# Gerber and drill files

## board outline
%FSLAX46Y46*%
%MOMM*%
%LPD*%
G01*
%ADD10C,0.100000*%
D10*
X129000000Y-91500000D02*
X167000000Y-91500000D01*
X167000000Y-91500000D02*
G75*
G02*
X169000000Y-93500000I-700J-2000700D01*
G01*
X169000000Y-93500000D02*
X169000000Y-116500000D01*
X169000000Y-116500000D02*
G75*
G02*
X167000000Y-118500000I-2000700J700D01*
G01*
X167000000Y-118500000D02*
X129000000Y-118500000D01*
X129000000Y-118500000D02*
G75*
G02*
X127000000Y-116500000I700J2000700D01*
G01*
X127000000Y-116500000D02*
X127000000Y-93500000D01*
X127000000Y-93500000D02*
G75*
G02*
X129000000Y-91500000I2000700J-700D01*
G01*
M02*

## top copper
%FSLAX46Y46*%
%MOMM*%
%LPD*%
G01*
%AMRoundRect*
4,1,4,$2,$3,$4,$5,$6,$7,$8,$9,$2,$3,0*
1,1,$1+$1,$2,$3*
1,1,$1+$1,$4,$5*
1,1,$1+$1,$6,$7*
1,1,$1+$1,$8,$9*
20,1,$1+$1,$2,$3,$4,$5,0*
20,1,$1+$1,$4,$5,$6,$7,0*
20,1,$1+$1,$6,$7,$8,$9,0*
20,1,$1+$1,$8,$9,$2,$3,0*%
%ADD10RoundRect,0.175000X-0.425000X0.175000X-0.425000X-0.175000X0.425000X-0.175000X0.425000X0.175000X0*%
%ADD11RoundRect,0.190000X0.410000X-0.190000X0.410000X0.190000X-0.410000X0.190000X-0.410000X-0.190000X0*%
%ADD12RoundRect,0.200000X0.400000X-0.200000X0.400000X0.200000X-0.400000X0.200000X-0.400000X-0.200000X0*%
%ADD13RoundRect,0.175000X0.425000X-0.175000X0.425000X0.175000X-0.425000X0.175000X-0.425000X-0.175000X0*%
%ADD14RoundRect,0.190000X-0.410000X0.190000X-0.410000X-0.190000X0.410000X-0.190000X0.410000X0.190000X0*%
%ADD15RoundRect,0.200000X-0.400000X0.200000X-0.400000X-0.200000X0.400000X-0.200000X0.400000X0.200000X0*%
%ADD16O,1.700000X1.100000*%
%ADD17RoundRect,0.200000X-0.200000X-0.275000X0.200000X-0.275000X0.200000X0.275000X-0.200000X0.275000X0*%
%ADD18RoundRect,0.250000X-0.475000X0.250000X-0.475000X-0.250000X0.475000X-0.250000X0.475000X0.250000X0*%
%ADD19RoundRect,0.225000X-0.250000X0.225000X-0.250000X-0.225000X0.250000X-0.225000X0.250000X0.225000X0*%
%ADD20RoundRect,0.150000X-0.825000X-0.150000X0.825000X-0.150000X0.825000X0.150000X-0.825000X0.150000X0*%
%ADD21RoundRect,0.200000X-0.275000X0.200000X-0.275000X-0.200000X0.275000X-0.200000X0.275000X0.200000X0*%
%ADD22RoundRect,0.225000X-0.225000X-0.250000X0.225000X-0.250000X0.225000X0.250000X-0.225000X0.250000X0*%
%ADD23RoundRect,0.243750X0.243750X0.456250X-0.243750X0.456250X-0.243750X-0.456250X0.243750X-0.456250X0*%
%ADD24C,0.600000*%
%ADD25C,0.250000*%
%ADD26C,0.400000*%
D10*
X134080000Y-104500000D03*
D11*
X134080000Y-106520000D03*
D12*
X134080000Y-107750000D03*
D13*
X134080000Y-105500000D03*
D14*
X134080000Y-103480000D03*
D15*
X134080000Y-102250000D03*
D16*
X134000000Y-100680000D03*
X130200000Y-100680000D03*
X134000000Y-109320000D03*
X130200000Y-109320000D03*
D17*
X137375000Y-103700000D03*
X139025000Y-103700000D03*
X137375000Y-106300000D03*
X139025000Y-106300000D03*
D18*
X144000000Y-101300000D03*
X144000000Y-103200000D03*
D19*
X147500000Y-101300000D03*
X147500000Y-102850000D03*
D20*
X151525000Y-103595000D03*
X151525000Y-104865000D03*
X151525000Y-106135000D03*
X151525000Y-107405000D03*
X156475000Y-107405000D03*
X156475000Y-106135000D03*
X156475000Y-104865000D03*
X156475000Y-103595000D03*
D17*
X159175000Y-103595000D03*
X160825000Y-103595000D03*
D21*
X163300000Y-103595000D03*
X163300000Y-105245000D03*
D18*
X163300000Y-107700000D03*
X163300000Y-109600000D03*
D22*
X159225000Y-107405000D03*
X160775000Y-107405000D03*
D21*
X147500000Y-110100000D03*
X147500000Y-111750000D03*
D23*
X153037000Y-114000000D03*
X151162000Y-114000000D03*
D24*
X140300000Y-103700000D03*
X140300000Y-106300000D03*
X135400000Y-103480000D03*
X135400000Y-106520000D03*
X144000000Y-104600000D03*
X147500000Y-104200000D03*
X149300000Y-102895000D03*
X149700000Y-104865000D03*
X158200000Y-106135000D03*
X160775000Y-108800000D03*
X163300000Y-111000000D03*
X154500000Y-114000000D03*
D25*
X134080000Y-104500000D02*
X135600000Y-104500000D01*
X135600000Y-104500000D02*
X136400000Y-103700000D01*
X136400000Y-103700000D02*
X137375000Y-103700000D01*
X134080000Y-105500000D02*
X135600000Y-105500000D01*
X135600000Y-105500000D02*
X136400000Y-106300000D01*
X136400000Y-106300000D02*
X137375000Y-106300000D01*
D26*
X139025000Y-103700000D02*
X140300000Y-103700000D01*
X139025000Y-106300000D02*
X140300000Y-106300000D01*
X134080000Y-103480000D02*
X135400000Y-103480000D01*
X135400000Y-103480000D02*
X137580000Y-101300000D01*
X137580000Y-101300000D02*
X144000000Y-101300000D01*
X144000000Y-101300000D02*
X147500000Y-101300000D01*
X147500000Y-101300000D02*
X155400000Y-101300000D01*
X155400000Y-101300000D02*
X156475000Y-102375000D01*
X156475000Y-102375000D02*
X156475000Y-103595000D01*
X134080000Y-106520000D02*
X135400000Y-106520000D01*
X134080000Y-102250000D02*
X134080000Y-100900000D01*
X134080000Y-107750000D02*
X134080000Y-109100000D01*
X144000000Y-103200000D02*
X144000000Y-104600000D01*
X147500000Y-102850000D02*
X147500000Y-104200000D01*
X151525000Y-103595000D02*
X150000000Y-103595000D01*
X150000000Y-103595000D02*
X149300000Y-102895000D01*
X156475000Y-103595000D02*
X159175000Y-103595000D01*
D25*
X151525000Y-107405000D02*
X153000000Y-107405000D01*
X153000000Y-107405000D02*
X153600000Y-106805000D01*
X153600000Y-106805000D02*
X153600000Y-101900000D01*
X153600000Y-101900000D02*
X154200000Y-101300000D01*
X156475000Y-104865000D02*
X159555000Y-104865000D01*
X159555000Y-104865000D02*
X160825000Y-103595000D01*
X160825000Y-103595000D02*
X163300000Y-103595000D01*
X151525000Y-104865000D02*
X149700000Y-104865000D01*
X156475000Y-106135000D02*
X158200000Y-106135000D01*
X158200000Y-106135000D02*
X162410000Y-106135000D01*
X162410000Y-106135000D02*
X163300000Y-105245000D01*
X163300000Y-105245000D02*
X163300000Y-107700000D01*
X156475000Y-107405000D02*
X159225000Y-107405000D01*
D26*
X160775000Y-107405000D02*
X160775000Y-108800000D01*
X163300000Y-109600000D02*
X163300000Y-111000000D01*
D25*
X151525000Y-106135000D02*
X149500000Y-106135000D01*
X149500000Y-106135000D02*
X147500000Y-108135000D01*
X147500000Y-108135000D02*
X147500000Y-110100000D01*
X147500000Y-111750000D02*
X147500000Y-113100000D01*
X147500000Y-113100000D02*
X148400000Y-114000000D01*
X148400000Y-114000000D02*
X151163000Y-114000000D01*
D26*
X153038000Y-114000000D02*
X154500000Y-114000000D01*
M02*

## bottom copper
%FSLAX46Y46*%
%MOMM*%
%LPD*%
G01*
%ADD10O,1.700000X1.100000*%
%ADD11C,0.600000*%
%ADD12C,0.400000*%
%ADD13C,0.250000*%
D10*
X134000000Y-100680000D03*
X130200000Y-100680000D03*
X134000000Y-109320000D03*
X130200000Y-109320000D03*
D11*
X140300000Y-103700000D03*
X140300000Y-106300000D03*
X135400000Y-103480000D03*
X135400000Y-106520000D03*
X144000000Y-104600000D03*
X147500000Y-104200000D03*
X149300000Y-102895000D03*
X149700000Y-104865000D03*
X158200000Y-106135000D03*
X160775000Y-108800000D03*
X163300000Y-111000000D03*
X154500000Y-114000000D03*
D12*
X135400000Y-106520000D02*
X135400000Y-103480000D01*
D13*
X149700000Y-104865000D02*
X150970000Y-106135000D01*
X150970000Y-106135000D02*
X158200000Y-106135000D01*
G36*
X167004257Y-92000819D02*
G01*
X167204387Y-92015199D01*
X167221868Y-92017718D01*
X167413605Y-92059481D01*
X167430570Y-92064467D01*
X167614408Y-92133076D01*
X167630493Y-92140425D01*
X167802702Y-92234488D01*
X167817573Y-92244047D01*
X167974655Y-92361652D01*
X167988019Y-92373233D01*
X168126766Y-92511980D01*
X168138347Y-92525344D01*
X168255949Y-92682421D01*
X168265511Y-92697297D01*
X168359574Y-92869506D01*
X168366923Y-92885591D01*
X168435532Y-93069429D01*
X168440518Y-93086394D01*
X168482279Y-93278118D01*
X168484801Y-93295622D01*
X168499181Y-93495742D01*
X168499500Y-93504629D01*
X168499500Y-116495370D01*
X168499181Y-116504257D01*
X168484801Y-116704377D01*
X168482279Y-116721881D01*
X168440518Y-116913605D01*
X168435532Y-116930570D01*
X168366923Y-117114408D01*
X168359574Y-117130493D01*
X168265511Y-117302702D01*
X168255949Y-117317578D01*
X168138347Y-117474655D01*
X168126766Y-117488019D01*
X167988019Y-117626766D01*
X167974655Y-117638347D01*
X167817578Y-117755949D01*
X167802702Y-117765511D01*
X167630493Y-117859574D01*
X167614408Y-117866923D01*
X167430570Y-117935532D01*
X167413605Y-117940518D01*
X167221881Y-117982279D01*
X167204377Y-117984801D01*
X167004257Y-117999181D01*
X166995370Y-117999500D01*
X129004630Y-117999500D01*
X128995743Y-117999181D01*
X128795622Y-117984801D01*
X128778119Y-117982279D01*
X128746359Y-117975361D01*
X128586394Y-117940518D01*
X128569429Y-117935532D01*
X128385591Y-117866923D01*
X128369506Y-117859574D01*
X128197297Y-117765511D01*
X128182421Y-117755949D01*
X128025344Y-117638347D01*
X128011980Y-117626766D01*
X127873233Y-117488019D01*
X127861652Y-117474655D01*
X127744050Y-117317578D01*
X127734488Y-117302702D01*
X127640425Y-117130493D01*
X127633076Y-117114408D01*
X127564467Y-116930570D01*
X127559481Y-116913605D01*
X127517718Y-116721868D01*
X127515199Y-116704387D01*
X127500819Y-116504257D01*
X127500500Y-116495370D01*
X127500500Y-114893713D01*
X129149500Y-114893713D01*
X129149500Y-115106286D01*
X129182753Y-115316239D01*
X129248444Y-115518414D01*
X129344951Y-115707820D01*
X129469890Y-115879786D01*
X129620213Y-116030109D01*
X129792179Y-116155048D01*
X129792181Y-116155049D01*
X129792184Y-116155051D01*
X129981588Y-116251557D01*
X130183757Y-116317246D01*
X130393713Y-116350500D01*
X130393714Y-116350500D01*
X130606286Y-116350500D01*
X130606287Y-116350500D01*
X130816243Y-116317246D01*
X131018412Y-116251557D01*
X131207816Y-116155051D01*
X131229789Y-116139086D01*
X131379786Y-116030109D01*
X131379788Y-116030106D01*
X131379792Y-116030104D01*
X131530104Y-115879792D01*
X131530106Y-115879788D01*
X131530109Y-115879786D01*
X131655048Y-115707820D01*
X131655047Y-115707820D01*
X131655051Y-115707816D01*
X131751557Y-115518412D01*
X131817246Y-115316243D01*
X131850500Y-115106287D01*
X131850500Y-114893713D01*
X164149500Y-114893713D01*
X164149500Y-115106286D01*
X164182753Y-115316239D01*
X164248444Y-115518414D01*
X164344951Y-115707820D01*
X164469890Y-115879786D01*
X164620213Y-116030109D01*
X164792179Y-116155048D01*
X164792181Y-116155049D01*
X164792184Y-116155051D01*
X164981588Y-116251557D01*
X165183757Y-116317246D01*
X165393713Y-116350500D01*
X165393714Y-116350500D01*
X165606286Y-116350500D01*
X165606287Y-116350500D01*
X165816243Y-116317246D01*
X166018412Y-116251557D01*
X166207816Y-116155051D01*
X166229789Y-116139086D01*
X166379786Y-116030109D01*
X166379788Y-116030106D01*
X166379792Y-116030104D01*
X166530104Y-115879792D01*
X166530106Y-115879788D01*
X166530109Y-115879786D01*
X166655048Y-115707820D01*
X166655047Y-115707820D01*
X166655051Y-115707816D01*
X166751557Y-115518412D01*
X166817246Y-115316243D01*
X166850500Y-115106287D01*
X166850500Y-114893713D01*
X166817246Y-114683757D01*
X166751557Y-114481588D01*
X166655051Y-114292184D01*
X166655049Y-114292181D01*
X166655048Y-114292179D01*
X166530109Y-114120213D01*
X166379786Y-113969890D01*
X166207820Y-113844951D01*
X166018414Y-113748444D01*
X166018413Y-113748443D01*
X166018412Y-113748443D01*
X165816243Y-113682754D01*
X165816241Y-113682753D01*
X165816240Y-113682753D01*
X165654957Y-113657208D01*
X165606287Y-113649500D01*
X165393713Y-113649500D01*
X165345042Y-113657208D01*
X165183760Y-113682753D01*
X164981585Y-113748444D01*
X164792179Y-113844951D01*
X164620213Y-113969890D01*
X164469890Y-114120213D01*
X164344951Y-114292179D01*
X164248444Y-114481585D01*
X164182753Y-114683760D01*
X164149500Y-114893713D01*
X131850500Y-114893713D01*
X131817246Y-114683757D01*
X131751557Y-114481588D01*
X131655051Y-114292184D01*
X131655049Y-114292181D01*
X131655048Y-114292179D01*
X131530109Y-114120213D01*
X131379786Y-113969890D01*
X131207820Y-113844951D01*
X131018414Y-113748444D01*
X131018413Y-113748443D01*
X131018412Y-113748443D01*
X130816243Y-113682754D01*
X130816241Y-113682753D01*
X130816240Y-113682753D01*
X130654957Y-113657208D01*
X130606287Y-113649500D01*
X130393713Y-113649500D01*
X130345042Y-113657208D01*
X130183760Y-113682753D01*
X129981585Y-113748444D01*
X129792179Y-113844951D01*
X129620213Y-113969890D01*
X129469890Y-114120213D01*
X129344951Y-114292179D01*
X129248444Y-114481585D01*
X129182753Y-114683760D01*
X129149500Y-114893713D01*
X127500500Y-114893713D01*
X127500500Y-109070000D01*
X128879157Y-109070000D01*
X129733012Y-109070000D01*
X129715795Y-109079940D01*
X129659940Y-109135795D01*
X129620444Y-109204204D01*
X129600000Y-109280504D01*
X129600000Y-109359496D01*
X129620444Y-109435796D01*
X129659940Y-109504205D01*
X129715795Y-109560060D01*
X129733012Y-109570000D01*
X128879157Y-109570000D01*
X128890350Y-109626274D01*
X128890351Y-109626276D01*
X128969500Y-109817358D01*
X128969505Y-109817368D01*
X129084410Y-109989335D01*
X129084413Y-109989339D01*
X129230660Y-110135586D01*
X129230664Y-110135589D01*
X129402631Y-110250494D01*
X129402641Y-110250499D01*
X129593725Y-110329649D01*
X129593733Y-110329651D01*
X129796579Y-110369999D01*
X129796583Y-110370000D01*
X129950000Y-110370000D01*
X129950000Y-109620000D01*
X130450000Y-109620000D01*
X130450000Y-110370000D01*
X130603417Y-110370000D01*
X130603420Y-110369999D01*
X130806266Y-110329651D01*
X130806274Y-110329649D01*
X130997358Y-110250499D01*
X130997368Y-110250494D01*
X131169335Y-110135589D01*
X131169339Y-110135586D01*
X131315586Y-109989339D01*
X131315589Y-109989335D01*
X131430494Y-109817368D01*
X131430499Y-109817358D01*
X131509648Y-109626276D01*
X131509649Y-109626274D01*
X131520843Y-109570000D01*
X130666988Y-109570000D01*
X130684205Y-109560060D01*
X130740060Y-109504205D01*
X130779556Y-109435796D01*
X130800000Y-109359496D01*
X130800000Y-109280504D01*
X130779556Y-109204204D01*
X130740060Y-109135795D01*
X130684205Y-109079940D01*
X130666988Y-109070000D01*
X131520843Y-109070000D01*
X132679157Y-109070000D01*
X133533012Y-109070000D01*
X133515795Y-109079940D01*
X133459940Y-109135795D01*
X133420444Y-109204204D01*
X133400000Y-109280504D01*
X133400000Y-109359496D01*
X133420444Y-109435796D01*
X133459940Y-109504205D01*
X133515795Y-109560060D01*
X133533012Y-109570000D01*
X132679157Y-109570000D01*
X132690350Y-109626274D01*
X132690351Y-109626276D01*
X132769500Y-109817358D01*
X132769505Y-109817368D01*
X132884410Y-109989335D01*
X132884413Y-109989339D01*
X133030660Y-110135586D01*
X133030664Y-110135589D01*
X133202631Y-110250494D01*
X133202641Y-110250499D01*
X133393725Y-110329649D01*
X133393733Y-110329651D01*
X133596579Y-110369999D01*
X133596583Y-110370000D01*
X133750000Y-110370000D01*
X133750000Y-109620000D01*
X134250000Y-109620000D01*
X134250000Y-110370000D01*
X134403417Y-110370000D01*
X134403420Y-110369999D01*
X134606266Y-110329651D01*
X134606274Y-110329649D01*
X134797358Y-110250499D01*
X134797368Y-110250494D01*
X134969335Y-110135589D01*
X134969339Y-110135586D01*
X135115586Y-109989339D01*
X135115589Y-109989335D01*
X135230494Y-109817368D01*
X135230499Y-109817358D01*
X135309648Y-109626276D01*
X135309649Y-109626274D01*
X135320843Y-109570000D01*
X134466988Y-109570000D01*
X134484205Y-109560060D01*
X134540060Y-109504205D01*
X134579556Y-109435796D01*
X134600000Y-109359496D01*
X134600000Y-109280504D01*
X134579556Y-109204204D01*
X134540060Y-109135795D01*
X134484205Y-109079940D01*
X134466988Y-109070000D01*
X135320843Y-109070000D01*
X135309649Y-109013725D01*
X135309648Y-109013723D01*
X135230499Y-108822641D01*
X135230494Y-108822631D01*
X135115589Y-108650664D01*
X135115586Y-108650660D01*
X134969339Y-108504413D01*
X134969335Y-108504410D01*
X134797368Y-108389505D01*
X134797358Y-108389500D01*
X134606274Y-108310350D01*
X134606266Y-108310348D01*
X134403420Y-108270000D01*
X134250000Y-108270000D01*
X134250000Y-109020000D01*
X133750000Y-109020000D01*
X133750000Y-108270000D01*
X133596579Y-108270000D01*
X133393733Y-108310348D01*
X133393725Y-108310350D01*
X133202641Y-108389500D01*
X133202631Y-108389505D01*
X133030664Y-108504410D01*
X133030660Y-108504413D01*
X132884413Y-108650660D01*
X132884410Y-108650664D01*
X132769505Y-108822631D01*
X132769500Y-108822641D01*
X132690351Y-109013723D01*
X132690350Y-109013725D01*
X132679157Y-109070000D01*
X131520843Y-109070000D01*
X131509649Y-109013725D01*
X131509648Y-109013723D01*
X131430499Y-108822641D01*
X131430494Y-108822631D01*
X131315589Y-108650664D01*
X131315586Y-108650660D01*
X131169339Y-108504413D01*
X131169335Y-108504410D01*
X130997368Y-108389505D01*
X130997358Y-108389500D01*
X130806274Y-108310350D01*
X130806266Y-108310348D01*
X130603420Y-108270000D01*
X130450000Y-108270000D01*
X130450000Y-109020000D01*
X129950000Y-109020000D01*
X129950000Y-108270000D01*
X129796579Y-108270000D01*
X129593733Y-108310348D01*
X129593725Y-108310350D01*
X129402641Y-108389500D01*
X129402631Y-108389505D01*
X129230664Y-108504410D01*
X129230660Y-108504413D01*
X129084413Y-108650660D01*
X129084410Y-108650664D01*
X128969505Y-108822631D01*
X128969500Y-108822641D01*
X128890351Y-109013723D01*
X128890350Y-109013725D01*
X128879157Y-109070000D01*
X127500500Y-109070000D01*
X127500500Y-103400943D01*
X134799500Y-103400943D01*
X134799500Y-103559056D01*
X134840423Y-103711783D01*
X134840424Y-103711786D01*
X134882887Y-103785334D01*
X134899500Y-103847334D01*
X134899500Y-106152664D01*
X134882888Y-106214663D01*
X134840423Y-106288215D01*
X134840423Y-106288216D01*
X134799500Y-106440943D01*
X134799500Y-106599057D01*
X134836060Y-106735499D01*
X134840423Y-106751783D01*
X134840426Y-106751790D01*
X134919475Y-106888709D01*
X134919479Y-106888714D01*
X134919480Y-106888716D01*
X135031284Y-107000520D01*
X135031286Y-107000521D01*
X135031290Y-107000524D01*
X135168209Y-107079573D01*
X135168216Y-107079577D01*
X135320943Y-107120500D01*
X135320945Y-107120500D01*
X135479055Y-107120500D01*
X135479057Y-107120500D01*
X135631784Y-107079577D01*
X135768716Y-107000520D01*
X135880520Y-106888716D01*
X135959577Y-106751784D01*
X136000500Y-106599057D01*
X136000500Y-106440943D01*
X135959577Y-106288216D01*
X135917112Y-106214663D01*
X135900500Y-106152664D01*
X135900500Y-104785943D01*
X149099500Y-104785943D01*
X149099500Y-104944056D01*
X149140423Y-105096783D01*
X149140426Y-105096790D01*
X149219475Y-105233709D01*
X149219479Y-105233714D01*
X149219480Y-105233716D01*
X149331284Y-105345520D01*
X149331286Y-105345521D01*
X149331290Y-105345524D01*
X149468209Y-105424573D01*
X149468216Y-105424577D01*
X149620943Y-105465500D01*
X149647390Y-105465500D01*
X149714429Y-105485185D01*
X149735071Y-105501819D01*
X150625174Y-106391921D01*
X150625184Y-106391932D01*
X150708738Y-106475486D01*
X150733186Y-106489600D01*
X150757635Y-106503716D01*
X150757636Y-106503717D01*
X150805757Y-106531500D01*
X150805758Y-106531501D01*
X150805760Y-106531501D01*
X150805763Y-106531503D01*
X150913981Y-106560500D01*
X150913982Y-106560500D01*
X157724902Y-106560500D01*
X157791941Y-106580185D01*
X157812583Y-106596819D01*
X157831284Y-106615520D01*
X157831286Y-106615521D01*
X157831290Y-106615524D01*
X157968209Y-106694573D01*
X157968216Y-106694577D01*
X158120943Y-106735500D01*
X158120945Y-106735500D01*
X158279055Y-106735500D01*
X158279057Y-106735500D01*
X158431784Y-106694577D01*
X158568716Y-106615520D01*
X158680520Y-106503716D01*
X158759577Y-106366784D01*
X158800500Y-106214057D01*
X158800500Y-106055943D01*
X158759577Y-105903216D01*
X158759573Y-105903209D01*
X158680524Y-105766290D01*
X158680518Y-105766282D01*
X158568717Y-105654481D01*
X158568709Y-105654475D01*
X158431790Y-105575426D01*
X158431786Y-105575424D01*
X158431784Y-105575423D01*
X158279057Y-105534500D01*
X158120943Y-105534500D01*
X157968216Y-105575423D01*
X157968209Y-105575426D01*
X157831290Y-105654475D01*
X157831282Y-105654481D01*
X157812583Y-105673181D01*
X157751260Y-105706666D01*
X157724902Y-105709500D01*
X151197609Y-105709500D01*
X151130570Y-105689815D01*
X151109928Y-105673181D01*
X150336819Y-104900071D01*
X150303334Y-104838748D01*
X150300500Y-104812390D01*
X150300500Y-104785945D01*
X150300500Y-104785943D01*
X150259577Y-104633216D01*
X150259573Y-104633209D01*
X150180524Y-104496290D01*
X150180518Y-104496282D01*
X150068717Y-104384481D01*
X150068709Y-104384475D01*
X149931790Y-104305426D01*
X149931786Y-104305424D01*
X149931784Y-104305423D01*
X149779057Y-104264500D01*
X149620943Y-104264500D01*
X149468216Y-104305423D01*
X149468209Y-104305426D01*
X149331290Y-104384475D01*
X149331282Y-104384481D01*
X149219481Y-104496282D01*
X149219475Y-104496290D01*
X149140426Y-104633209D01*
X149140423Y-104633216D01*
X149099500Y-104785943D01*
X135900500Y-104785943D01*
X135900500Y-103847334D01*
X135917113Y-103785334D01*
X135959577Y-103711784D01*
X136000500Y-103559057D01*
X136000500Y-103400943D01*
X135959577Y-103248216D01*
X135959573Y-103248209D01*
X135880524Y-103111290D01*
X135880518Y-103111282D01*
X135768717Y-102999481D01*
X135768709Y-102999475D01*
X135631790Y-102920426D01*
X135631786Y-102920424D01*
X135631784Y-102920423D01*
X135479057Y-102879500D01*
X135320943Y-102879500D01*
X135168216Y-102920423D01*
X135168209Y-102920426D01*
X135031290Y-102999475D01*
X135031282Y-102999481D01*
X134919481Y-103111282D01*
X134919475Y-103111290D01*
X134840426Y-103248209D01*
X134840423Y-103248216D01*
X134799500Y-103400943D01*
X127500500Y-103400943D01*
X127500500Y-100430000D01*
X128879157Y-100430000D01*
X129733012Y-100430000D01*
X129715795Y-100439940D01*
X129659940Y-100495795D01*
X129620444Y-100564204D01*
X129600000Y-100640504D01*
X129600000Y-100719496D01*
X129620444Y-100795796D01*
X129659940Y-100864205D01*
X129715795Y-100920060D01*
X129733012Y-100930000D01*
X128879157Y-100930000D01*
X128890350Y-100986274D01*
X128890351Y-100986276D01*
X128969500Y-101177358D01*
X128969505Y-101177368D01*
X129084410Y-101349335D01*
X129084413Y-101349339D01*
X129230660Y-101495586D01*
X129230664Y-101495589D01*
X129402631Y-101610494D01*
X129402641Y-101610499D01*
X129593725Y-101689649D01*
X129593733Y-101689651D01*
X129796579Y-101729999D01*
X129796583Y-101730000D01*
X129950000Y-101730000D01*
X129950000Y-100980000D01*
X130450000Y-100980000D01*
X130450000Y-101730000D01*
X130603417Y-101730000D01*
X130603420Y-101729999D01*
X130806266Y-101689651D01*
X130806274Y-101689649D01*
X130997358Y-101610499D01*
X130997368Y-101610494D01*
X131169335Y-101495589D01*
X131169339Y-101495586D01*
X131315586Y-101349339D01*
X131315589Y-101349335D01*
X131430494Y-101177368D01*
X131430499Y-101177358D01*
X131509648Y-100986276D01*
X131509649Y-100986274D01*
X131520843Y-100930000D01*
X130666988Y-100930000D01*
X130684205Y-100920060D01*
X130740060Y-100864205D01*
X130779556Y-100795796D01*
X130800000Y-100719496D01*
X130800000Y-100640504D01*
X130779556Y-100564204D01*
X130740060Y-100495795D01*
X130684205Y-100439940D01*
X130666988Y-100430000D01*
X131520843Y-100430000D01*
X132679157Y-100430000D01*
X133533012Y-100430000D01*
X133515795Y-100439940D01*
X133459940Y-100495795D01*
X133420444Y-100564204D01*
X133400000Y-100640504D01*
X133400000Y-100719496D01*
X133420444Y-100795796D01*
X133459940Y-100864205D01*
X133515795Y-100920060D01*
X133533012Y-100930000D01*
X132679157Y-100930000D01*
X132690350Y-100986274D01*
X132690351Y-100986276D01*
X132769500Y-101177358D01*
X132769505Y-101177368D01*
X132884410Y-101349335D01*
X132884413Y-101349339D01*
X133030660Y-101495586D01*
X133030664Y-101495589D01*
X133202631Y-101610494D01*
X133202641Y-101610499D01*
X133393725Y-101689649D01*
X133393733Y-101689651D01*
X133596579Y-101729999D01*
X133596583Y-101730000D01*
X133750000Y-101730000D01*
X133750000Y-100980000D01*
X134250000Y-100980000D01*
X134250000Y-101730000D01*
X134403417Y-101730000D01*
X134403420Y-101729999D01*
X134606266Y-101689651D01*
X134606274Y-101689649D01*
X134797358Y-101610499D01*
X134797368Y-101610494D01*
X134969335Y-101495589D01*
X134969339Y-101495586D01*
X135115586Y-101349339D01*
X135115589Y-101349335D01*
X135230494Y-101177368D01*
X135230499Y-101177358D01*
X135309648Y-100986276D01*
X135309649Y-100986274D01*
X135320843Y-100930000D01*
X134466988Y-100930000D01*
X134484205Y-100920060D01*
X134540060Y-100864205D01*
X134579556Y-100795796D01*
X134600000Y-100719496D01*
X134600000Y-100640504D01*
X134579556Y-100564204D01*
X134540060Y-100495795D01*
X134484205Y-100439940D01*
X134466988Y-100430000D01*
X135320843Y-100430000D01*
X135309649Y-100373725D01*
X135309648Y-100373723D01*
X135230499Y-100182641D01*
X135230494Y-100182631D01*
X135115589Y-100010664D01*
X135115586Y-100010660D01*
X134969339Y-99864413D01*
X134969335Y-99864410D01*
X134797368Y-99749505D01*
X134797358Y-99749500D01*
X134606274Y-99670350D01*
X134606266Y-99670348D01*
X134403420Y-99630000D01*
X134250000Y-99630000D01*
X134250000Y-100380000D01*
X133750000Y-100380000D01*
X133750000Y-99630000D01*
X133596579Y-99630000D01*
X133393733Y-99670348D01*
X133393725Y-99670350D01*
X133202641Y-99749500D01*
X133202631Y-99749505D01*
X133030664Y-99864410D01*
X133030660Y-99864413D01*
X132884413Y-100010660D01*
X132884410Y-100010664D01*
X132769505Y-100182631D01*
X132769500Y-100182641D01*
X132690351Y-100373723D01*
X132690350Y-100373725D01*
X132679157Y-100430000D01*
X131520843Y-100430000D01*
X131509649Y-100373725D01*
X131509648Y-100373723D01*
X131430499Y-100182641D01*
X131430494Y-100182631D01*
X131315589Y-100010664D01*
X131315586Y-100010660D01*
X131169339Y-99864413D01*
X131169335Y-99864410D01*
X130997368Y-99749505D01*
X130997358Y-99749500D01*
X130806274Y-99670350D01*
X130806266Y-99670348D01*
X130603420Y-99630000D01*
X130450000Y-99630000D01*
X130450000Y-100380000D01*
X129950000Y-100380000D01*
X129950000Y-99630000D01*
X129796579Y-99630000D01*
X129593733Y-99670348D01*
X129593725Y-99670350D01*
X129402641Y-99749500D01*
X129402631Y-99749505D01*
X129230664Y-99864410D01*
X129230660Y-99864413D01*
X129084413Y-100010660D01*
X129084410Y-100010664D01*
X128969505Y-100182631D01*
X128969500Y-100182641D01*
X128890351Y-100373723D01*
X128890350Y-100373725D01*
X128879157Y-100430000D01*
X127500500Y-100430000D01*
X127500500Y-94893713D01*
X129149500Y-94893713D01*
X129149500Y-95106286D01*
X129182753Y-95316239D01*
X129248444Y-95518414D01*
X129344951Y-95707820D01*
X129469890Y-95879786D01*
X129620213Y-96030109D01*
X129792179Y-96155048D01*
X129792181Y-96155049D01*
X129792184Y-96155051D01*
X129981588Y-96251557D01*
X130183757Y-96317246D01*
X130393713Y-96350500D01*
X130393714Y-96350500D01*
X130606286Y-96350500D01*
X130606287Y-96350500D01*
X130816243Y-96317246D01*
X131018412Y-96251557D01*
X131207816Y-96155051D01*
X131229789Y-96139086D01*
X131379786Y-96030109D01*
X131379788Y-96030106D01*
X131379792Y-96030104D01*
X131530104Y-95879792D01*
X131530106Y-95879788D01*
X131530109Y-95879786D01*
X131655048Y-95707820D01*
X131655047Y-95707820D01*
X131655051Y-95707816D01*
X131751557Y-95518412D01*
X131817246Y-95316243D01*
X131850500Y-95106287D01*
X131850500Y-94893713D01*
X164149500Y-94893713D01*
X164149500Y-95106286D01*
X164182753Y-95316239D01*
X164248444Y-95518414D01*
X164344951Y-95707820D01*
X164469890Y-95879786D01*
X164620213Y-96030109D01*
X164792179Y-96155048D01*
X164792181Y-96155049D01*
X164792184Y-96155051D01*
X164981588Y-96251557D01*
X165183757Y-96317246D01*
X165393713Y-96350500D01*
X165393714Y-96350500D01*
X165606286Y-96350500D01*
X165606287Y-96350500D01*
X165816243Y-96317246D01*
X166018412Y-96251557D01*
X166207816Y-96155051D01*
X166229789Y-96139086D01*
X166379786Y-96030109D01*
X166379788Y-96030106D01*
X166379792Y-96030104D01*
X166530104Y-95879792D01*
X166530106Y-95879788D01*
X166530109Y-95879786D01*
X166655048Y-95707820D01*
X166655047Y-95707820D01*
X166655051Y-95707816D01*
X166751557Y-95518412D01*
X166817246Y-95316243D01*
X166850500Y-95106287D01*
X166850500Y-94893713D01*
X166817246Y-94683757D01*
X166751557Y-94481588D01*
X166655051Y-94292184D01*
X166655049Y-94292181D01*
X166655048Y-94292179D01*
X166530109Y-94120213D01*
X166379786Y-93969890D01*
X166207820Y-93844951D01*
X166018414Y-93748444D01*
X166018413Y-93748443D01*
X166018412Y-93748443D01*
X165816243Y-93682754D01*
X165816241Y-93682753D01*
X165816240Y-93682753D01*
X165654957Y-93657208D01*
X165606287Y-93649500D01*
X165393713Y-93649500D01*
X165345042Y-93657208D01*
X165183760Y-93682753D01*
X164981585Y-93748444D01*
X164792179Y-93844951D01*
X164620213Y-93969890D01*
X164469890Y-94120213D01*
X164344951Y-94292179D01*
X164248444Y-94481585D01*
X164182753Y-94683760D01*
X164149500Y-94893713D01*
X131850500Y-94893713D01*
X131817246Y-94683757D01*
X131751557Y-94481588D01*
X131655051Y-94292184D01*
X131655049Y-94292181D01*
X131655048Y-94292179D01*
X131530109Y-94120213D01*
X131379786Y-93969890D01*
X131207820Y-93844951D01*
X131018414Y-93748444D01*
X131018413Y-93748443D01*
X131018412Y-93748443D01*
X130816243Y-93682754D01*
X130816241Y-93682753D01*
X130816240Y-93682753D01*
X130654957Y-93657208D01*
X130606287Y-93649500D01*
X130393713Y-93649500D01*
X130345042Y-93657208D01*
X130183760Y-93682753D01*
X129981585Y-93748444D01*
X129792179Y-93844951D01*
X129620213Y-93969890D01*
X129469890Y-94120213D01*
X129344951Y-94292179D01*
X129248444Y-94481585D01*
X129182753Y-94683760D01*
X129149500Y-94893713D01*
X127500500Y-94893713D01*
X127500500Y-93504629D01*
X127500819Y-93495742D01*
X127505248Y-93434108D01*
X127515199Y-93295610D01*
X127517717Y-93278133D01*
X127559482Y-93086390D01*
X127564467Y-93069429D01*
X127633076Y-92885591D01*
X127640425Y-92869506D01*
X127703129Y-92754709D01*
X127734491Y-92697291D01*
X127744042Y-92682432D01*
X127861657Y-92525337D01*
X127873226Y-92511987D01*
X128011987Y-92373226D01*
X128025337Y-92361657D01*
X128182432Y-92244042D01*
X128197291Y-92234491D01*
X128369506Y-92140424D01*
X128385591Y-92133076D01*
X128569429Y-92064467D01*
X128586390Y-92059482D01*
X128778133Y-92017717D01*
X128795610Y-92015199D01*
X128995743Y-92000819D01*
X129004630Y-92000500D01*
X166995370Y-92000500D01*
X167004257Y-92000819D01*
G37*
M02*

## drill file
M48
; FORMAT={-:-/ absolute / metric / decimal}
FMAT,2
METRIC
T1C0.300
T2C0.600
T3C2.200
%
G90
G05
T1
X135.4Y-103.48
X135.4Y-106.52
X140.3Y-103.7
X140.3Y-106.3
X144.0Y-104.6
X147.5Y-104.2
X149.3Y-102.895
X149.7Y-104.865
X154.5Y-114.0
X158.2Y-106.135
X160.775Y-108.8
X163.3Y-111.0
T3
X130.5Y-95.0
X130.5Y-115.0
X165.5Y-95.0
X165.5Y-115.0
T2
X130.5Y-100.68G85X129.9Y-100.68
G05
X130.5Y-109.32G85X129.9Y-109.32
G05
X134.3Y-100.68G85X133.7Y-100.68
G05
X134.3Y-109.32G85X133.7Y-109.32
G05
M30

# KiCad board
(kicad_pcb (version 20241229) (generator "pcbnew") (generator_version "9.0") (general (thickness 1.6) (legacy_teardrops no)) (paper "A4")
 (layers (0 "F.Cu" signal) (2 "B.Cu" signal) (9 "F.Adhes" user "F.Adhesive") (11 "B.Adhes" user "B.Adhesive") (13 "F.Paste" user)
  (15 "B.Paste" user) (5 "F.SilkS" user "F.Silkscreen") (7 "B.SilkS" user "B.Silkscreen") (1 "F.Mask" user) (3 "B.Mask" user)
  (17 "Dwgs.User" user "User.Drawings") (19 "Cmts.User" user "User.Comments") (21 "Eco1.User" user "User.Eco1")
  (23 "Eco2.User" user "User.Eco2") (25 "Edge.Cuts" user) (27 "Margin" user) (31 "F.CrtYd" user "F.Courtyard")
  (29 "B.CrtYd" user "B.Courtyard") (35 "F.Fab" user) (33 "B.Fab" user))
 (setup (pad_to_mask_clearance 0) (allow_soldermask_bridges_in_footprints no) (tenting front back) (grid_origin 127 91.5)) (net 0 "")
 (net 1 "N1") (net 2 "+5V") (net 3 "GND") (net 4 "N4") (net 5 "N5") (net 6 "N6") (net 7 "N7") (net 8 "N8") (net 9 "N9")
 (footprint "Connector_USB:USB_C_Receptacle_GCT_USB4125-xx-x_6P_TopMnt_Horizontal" (layer "F.Cu") (at 131 105 270)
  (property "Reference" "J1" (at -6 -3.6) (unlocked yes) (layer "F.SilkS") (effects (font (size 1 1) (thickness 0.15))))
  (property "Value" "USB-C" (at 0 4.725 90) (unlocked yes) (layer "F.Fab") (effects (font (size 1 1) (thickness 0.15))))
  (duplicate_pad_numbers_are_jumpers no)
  (pad "A5" smd roundrect (at -0.5 -3.08 270) (size 0.7 1.2) (layers "F.Cu" "F.Mask" "F.Paste") (roundrect_rratio 0.25) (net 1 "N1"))
  (pad "A9" smd roundrect (at 1.52 -3.08 90) (size 0.76 1.2) (layers "F.Cu" "F.Mask" "F.Paste") (roundrect_rratio 0.25) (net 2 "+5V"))
  (pad "A12" smd roundrect (at 2.75 -3.08 90) (size 0.8 1.2) (layers "F.Cu" "F.Mask" "F.Paste") (roundrect_rratio 0.25) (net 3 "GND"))
  (pad "B5" smd roundrect (at 0.5 -3.08 90) (size 0.7 1.2) (layers "F.Cu" "F.Mask" "F.Paste") (roundrect_rratio 0.25) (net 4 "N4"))
  (pad "B9" smd roundrect (at -1.52 -3.08 270) (size 0.76 1.2) (layers "F.Cu" "F.Mask" "F.Paste") (roundrect_rratio 0.25) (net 2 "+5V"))
  (pad "B12" smd roundrect (at -2.75 -3.08 270) (size 0.8 1.2) (layers "F.Cu" "F.Mask" "F.Paste") (roundrect_rratio 0.25) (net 3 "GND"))
  (pad "SH" thru_hole oval (at -4.32 -3 270) (size 1.1 1.7) (drill oval 0.6 1.2) (layers "*.Cu" "*.Mask" "F.Paste")
   (remove_unused_layers no) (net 3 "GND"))
  (pad "SH" thru_hole oval (at -4.32 0.8 270) (size 1.1 1.7) (drill oval 0.6 1.2) (layers "*.Cu" "*.Mask" "F.Paste")
   (remove_unused_layers no) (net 3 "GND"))
  (pad "SH" thru_hole oval (at 4.32 -3 270) (size 1.1 1.7) (drill oval 0.6 1.2) (layers "*.Cu" "*.Mask" "F.Paste") (remove_unused_layers no)
   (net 3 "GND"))
  (pad "SH" thru_hole oval (at 4.32 0.8 270) (size 1.1 1.7) (drill oval 0.6 1.2) (layers "*.Cu" "*.Mask" "F.Paste")
   (remove_unused_layers no) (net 3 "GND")))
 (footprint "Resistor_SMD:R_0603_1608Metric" (layer "F.Cu") (at 138.2 103.7)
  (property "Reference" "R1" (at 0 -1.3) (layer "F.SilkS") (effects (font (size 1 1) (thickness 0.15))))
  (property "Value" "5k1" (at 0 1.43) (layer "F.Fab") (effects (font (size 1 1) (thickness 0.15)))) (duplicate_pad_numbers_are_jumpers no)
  (pad "1" smd roundrect (at -0.825 0) (size 0.8 0.95) (layers "F.Cu" "F.Mask" "F.Paste") (roundrect_rratio 0.25) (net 1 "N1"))
  (pad "2" smd roundrect (at 0.825 0) (size 0.8 0.95) (layers "F.Cu" "F.Mask" "F.Paste") (roundrect_rratio 0.25) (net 3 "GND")))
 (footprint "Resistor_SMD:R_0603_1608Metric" (layer "F.Cu") (at 138.2 106.3)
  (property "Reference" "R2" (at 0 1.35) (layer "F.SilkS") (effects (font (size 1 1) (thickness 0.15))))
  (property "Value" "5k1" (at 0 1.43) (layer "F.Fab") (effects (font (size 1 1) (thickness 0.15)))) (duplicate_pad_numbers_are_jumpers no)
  (pad "1" smd roundrect (at -0.825 0) (size 0.8 0.95) (layers "F.Cu" "F.Mask" "F.Paste") (roundrect_rratio 0.25) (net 4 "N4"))
  (pad "2" smd roundrect (at 0.825 0) (size 0.8 0.95) (layers "F.Cu" "F.Mask" "F.Paste") (roundrect_rratio 0.25) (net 3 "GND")))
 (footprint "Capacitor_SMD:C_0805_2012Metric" (layer "F.Cu") (at 144 102.25 270)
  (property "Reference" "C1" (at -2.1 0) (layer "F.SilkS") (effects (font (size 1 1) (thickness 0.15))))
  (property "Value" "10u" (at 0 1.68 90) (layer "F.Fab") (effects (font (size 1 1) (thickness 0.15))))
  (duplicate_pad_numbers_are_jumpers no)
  (pad "1" smd roundrect (at -0.95 0 270) (size 1 1.45) (layers "F.Cu" "F.Mask" "F.Paste") (roundrect_rratio 0.25) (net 2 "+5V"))
  (pad "2" smd roundrect (at 0.95 0 270) (size 1 1.45) (layers "F.Cu" "F.Mask" "F.Paste") (roundrect_rratio 0.25) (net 3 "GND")))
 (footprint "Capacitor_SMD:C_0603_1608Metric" (layer "F.Cu") (at 147.5 102.075 270)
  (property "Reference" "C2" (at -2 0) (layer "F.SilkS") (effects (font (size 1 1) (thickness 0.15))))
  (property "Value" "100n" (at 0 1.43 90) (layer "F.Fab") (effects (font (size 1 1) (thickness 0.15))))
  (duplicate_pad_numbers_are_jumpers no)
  (pad "1" smd roundrect (at -0.775 0 270) (size 0.9 0.95) (layers "F.Cu" "F.Mask" "F.Paste") (roundrect_rratio 0.25) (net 2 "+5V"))
  (pad "2" smd roundrect (at 0.775 0 270) (size 0.9 0.95) (layers "F.Cu" "F.Mask" "F.Paste") (roundrect_rratio 0.25) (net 3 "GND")))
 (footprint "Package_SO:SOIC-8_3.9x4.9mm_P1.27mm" (layer "F.Cu") (at 154 105.5)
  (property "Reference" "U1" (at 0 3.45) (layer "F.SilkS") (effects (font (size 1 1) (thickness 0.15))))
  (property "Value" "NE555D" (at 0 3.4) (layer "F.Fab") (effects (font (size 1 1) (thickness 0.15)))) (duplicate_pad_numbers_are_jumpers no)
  (pad "1" smd roundrect (at -2.475 -1.905) (size 1.95 0.6) (layers "F.Cu" "F.Mask" "F.Paste") (roundrect_rratio 0.25) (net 3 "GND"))
  (pad "2" smd roundrect (at -2.475 -0.635) (size 1.95 0.6) (layers "F.Cu" "F.Mask" "F.Paste") (roundrect_rratio 0.25) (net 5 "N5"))
  (pad "3" smd roundrect (at -2.475 0.635) (size 1.95 0.6) (layers "F.Cu" "F.Mask" "F.Paste") (roundrect_rratio 0.25) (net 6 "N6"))
  (pad "4" smd roundrect (at -2.475 1.905) (size 1.95 0.6) (layers "F.Cu" "F.Mask" "F.Paste") (roundrect_rratio 0.25) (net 2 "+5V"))
  (pad "5" smd roundrect (at 2.475 1.905) (size 1.95 0.6) (layers "F.Cu" "F.Mask" "F.Paste") (roundrect_rratio 0.25) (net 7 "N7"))
  (pad "6" smd roundrect (at 2.475 0.635) (size 1.95 0.6) (layers "F.Cu" "F.Mask" "F.Paste") (roundrect_rratio 0.25) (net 5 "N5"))
  (pad "7" smd roundrect (at 2.475 -0.635) (size 1.95 0.6) (layers "F.Cu" "F.Mask" "F.Paste") (roundrect_rratio 0.25) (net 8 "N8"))
  (pad "8" smd roundrect (at 2.475 -1.905) (size 1.95 0.6) (layers "F.Cu" "F.Mask" "F.Paste") (roundrect_rratio 0.25) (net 2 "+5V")))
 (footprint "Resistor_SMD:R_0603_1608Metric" (layer "F.Cu") (at 160 103.595)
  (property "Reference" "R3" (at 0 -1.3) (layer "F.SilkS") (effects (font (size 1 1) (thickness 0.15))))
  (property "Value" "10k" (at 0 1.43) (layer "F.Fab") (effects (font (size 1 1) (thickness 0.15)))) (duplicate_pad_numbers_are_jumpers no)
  (pad "1" smd roundrect (at -0.825 0) (size 0.8 0.95) (layers "F.Cu" "F.Mask" "F.Paste") (roundrect_rratio 0.25) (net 2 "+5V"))
  (pad "2" smd roundrect (at 0.825 0) (size 0.8 0.95) (layers "F.Cu" "F.Mask" "F.Paste") (roundrect_rratio 0.25) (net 8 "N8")))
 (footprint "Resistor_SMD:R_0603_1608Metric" (layer "F.Cu") (at 163.3 104.42 270)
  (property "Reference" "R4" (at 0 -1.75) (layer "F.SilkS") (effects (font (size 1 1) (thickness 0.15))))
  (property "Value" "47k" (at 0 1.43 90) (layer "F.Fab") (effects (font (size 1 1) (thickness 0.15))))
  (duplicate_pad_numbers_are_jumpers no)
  (pad "1" smd roundrect (at -0.825 0 270) (size 0.8 0.95) (layers "F.Cu" "F.Mask" "F.Paste") (roundrect_rratio 0.25) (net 8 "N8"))
  (pad "2" smd roundrect (at 0.825 0 270) (size 0.8 0.95) (layers "F.Cu" "F.Mask" "F.Paste") (roundrect_rratio 0.25) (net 5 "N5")))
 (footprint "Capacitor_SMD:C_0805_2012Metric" (layer "F.Cu") (at 163.3 108.65 270)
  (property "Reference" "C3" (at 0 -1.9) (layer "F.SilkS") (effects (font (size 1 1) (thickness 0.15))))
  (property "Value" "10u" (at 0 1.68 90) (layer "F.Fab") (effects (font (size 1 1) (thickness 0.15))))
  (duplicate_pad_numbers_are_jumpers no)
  (pad "1" smd roundrect (at -0.95 0 270) (size 1 1.45) (layers "F.Cu" "F.Mask" "F.Paste") (roundrect_rratio 0.25) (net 5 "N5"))
  (pad "2" smd roundrect (at 0.95 0 270) (size 1 1.45) (layers "F.Cu" "F.Mask" "F.Paste") (roundrect_rratio 0.25) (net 3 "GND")))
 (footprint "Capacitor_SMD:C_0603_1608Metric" (layer "F.Cu") (at 160 107.405)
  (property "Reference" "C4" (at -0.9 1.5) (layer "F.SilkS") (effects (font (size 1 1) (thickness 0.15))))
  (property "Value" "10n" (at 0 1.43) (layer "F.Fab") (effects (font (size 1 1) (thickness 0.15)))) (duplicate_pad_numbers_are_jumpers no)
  (pad "1" smd roundrect (at -0.775 0) (size 0.9 0.95) (layers "F.Cu" "F.Mask" "F.Paste") (roundrect_rratio 0.25) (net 7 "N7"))
  (pad "2" smd roundrect (at 0.775 0) (size 0.9 0.95) (layers "F.Cu" "F.Mask" "F.Paste") (roundrect_rratio 0.25) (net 3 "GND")))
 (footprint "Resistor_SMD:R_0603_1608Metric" (layer "F.Cu") (at 147.5 110.925 270)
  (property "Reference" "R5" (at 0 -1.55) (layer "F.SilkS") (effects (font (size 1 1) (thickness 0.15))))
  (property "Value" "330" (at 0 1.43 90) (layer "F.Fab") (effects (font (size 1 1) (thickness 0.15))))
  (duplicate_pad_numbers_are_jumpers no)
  (pad "1" smd roundrect (at -0.825 0 270) (size 0.8 0.95) (layers "F.Cu" "F.Mask" "F.Paste") (roundrect_rratio 0.25) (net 6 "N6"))
  (pad "2" smd roundrect (at 0.825 0 270) (size 0.8 0.95) (layers "F.Cu" "F.Mask" "F.Paste") (roundrect_rratio 0.25) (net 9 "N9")))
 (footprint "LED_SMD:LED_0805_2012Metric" (layer "F.Cu") (at 152.1 114 180)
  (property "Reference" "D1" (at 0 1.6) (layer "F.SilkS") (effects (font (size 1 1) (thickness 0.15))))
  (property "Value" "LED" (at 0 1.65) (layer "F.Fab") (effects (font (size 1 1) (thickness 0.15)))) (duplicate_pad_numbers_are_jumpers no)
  (pad "1" smd roundrect (at -0.937 0 180) (size 0.975 1.4) (layers "F.Cu" "F.Mask" "F.Paste") (roundrect_rratio 0.25) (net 3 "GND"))
  (pad "2" smd roundrect (at 0.938 0 180) (size 0.975 1.4) (layers "F.Cu" "F.Mask" "F.Paste") (roundrect_rratio 0.25) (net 9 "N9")))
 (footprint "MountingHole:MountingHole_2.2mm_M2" (layer "F.Cu") (at 130.5 95)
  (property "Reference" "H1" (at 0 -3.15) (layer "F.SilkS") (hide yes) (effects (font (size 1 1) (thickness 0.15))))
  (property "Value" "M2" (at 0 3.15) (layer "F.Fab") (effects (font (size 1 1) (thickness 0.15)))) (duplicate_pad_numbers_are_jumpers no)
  (pad "" np_thru_hole circle (at 0 0) (size 2.2 2.2) (drill 2.2) (layers "*.Cu" "*.Mask")))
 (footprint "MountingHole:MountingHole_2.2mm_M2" (layer "F.Cu") (at 165.5 95)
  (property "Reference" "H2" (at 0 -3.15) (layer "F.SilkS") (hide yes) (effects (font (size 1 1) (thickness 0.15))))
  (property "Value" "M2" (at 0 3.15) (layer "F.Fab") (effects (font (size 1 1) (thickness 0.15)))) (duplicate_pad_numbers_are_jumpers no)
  (pad "" np_thru_hole circle (at 0 0) (size 2.2 2.2) (drill 2.2) (layers "*.Cu" "*.Mask")))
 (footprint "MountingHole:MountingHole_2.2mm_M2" (layer "F.Cu") (at 130.5 115)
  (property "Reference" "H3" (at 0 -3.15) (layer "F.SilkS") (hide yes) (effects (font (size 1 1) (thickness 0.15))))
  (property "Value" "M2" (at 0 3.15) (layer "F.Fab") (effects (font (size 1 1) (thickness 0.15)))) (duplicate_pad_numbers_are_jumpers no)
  (pad "" np_thru_hole circle (at 0 0) (size 2.2 2.2) (drill 2.2) (layers "*.Cu" "*.Mask")))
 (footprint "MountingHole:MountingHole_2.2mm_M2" (layer "F.Cu") (at 165.5 115)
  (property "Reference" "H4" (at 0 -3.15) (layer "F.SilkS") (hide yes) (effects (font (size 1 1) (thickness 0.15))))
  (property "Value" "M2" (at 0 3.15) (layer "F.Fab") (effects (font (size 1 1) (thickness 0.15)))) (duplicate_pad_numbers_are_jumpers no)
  (pad "" np_thru_hole circle (at 0 0) (size 2.2 2.2) (drill 2.2) (layers "*.Cu" "*.Mask")))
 (segment (start 134.08 104.5) (end 135.6 104.5) (width 0.25) (layer "F.Cu") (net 1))
 (segment (start 135.6 104.5) (end 136.4 103.7) (width 0.25) (layer "F.Cu") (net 1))
 (segment (start 136.4 103.7) (end 137.375 103.7) (width 0.25) (layer "F.Cu") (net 1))
 (segment (start 134.08 105.5) (end 135.6 105.5) (width 0.25) (layer "F.Cu") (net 4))
 (segment (start 135.6 105.5) (end 136.4 106.3) (width 0.25) (layer "F.Cu") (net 4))
 (segment (start 136.4 106.3) (end 137.375 106.3) (width 0.25) (layer "F.Cu") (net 4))
 (segment (start 139.025 103.7) (end 140.3 103.7) (width 0.4) (layer "F.Cu") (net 3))
 (via (at 140.3 103.7) (size 0.6) (drill 0.3) (layers "F.Cu" "B.Cu") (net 3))
 (segment (start 139.025 106.3) (end 140.3 106.3) (width 0.4) (layer "F.Cu") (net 3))
 (via (at 140.3 106.3) (size 0.6) (drill 0.3) (layers "F.Cu" "B.Cu") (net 3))
 (segment (start 134.08 103.48) (end 135.4 103.48) (width 0.4) (layer "F.Cu") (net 2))
 (via (at 135.4 103.48) (size 0.6) (drill 0.3) (layers "F.Cu" "B.Cu") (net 2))
 (segment (start 135.4 103.48) (end 137.58 101.3) (width 0.4) (layer "F.Cu") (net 2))
 (segment (start 137.58 101.3) (end 144 101.3) (width 0.4) (layer "F.Cu") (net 2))
 (segment (start 144 101.3) (end 147.5 101.3) (width 0.4) (layer "F.Cu") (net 2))
 (segment (start 147.5 101.3) (end 155.4 101.3) (width 0.4) (layer "F.Cu") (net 2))
 (segment (start 155.4 101.3) (end 156.475 102.375) (width 0.4) (layer "F.Cu") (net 2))
 (segment (start 156.475 102.375) (end 156.475 103.595) (width 0.4) (layer "F.Cu") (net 2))
 (segment (start 134.08 106.52) (end 135.4 106.52) (width 0.4) (layer "F.Cu") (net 2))
 (via (at 135.4 106.52) (size 0.6) (drill 0.3) (layers "F.Cu" "B.Cu") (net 2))
 (segment (start 135.4 106.52) (end 135.4 103.48) (width 0.4) (layer "B.Cu") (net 2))
 (segment (start 134.08 102.25) (end 134.08 100.9) (width 0.4) (layer "F.Cu") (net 3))
 (segment (start 134.08 107.75) (end 134.08 109.1) (width 0.4) (layer "F.Cu") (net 3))
 (segment (start 144 103.2) (end 144 104.6) (width 0.4) (layer "F.Cu") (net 3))
 (via (at 144 104.6) (size 0.6) (drill 0.3) (layers "F.Cu" "B.Cu") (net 3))
 (segment (start 147.5 102.85) (end 147.5 104.2) (width 0.4) (layer "F.Cu") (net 3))
 (via (at 147.5 104.2) (size 0.6) (drill 0.3) (layers "F.Cu" "B.Cu") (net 3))
 (segment (start 151.525 103.595) (end 150 103.595) (width 0.4) (layer "F.Cu") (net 3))
 (segment (start 150 103.595) (end 149.3 102.895) (width 0.4) (layer "F.Cu") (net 3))
 (via (at 149.3 102.895) (size 0.6) (drill 0.3) (layers "F.Cu" "B.Cu") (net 3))
 (segment (start 156.475 103.595) (end 159.175 103.595) (width 0.4) (layer "F.Cu") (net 2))
 (segment (start 151.525 107.405) (end 153 107.405) (width 0.25) (layer "F.Cu") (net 2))
 (segment (start 153 107.405) (end 153.6 106.805) (width 0.25) (layer "F.Cu") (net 2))
 (segment (start 153.6 106.805) (end 153.6 101.9) (width 0.25) (layer "F.Cu") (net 2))
 (segment (start 153.6 101.9) (end 154.2 101.3) (width 0.25) (layer "F.Cu") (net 2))
 (segment (start 156.475 104.865) (end 159.555 104.865) (width 0.25) (layer "F.Cu") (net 8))
 (segment (start 159.555 104.865) (end 160.825 103.595) (width 0.25) (layer "F.Cu") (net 8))
 (segment (start 160.825 103.595) (end 163.3 103.595) (width 0.25) (layer "F.Cu") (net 8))
 (segment (start 151.525 104.865) (end 149.7 104.865) (width 0.25) (layer "F.Cu") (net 5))
 (via (at 149.7 104.865) (size 0.6) (drill 0.3) (layers "F.Cu" "B.Cu") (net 5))
 (segment (start 149.7 104.865) (end 150.97 106.135) (width 0.25) (layer "B.Cu") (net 5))
 (segment (start 150.97 106.135) (end 158.2 106.135) (width 0.25) (layer "B.Cu") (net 5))
 (via (at 158.2 106.135) (size 0.6) (drill 0.3) (layers "F.Cu" "B.Cu") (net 5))
 (segment (start 156.475 106.135) (end 158.2 106.135) (width 0.25) (layer "F.Cu") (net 5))
 (segment (start 158.2 106.135) (end 162.41 106.135) (width 0.25) (layer "F.Cu") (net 5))
 (segment (start 162.41 106.135) (end 163.3 105.245) (width 0.25) (layer "F.Cu") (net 5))
 (segment (start 163.3 105.245) (end 163.3 107.7) (width 0.25) (layer "F.Cu") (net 5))
 (segment (start 156.475 107.405) (end 159.225 107.405) (width 0.25) (layer "F.Cu") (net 7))
 (segment (start 160.775 107.405) (end 160.775 108.8) (width 0.4) (layer "F.Cu") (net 3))
 (via (at 160.775 108.8) (size 0.6) (drill 0.3) (layers "F.Cu" "B.Cu") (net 3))
 (segment (start 163.3 109.6) (end 163.3 111) (width 0.4) (layer "F.Cu") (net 3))
 (via (at 163.3 111) (size 0.6) (drill 0.3) (layers "F.Cu" "B.Cu") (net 3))
 (segment (start 151.525 106.135) (end 149.5 106.135) (width 0.25) (layer "F.Cu") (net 6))
 (segment (start 149.5 106.135) (end 147.5 108.135) (width 0.25) (layer "F.Cu") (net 6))
 (segment (start 147.5 108.135) (end 147.5 110.1) (width 0.25) (layer "F.Cu") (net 6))
 (segment (start 147.5 111.75) (end 147.5 113.1) (width 0.25) (layer "F.Cu") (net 9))
 (segment (start 147.5 113.1) (end 148.4 114) (width 0.25) (layer "F.Cu") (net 9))
 (segment (start 148.4 114) (end 151.163 114) (width 0.25) (layer "F.Cu") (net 9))
 (segment (start 153.038 114) (end 154.5 114) (width 0.4) (layer "F.Cu") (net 3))
 (via (at 154.5 114) (size 0.6) (drill 0.3) (layers "F.Cu" "B.Cu") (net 3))
 (gr_line (start 129 91.5) (end 167 91.5) (stroke (width 0.1) (type default)) (layer "Edge.Cuts"))
 (gr_arc (start 167 91.5) (mid 168.414 92.086) (end 169 93.5) (stroke (width 0.1) (type default)) (layer "Edge.Cuts"))
 (gr_line (start 169 93.5) (end 169 116.5) (stroke (width 0.1) (type default)) (layer "Edge.Cuts"))
 (gr_arc (start 169 116.5) (mid 168.414 117.914) (end 167 118.5) (stroke (width 0.1) (type default)) (layer "Edge.Cuts"))
 (gr_line (start 167 118.5) (end 129 118.5) (stroke (width 0.1) (type default)) (layer "Edge.Cuts"))
 (gr_arc (start 129 118.5) (mid 127.586 117.914) (end 127 116.5) (stroke (width 0.1) (type default)) (layer "Edge.Cuts"))
 (gr_line (start 127 116.5) (end 127 93.5) (stroke (width 0.1) (type default)) (layer "Edge.Cuts"))
 (gr_arc (start 127 93.5) (mid 127.586 92.086) (end 129 91.5) (stroke (width 0.1) (type default)) (layer "Edge.Cuts"))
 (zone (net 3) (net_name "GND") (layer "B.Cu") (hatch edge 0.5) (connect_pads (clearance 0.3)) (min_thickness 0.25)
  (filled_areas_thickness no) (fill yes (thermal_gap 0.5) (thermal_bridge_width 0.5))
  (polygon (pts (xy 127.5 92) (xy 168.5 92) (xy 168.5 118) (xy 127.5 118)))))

